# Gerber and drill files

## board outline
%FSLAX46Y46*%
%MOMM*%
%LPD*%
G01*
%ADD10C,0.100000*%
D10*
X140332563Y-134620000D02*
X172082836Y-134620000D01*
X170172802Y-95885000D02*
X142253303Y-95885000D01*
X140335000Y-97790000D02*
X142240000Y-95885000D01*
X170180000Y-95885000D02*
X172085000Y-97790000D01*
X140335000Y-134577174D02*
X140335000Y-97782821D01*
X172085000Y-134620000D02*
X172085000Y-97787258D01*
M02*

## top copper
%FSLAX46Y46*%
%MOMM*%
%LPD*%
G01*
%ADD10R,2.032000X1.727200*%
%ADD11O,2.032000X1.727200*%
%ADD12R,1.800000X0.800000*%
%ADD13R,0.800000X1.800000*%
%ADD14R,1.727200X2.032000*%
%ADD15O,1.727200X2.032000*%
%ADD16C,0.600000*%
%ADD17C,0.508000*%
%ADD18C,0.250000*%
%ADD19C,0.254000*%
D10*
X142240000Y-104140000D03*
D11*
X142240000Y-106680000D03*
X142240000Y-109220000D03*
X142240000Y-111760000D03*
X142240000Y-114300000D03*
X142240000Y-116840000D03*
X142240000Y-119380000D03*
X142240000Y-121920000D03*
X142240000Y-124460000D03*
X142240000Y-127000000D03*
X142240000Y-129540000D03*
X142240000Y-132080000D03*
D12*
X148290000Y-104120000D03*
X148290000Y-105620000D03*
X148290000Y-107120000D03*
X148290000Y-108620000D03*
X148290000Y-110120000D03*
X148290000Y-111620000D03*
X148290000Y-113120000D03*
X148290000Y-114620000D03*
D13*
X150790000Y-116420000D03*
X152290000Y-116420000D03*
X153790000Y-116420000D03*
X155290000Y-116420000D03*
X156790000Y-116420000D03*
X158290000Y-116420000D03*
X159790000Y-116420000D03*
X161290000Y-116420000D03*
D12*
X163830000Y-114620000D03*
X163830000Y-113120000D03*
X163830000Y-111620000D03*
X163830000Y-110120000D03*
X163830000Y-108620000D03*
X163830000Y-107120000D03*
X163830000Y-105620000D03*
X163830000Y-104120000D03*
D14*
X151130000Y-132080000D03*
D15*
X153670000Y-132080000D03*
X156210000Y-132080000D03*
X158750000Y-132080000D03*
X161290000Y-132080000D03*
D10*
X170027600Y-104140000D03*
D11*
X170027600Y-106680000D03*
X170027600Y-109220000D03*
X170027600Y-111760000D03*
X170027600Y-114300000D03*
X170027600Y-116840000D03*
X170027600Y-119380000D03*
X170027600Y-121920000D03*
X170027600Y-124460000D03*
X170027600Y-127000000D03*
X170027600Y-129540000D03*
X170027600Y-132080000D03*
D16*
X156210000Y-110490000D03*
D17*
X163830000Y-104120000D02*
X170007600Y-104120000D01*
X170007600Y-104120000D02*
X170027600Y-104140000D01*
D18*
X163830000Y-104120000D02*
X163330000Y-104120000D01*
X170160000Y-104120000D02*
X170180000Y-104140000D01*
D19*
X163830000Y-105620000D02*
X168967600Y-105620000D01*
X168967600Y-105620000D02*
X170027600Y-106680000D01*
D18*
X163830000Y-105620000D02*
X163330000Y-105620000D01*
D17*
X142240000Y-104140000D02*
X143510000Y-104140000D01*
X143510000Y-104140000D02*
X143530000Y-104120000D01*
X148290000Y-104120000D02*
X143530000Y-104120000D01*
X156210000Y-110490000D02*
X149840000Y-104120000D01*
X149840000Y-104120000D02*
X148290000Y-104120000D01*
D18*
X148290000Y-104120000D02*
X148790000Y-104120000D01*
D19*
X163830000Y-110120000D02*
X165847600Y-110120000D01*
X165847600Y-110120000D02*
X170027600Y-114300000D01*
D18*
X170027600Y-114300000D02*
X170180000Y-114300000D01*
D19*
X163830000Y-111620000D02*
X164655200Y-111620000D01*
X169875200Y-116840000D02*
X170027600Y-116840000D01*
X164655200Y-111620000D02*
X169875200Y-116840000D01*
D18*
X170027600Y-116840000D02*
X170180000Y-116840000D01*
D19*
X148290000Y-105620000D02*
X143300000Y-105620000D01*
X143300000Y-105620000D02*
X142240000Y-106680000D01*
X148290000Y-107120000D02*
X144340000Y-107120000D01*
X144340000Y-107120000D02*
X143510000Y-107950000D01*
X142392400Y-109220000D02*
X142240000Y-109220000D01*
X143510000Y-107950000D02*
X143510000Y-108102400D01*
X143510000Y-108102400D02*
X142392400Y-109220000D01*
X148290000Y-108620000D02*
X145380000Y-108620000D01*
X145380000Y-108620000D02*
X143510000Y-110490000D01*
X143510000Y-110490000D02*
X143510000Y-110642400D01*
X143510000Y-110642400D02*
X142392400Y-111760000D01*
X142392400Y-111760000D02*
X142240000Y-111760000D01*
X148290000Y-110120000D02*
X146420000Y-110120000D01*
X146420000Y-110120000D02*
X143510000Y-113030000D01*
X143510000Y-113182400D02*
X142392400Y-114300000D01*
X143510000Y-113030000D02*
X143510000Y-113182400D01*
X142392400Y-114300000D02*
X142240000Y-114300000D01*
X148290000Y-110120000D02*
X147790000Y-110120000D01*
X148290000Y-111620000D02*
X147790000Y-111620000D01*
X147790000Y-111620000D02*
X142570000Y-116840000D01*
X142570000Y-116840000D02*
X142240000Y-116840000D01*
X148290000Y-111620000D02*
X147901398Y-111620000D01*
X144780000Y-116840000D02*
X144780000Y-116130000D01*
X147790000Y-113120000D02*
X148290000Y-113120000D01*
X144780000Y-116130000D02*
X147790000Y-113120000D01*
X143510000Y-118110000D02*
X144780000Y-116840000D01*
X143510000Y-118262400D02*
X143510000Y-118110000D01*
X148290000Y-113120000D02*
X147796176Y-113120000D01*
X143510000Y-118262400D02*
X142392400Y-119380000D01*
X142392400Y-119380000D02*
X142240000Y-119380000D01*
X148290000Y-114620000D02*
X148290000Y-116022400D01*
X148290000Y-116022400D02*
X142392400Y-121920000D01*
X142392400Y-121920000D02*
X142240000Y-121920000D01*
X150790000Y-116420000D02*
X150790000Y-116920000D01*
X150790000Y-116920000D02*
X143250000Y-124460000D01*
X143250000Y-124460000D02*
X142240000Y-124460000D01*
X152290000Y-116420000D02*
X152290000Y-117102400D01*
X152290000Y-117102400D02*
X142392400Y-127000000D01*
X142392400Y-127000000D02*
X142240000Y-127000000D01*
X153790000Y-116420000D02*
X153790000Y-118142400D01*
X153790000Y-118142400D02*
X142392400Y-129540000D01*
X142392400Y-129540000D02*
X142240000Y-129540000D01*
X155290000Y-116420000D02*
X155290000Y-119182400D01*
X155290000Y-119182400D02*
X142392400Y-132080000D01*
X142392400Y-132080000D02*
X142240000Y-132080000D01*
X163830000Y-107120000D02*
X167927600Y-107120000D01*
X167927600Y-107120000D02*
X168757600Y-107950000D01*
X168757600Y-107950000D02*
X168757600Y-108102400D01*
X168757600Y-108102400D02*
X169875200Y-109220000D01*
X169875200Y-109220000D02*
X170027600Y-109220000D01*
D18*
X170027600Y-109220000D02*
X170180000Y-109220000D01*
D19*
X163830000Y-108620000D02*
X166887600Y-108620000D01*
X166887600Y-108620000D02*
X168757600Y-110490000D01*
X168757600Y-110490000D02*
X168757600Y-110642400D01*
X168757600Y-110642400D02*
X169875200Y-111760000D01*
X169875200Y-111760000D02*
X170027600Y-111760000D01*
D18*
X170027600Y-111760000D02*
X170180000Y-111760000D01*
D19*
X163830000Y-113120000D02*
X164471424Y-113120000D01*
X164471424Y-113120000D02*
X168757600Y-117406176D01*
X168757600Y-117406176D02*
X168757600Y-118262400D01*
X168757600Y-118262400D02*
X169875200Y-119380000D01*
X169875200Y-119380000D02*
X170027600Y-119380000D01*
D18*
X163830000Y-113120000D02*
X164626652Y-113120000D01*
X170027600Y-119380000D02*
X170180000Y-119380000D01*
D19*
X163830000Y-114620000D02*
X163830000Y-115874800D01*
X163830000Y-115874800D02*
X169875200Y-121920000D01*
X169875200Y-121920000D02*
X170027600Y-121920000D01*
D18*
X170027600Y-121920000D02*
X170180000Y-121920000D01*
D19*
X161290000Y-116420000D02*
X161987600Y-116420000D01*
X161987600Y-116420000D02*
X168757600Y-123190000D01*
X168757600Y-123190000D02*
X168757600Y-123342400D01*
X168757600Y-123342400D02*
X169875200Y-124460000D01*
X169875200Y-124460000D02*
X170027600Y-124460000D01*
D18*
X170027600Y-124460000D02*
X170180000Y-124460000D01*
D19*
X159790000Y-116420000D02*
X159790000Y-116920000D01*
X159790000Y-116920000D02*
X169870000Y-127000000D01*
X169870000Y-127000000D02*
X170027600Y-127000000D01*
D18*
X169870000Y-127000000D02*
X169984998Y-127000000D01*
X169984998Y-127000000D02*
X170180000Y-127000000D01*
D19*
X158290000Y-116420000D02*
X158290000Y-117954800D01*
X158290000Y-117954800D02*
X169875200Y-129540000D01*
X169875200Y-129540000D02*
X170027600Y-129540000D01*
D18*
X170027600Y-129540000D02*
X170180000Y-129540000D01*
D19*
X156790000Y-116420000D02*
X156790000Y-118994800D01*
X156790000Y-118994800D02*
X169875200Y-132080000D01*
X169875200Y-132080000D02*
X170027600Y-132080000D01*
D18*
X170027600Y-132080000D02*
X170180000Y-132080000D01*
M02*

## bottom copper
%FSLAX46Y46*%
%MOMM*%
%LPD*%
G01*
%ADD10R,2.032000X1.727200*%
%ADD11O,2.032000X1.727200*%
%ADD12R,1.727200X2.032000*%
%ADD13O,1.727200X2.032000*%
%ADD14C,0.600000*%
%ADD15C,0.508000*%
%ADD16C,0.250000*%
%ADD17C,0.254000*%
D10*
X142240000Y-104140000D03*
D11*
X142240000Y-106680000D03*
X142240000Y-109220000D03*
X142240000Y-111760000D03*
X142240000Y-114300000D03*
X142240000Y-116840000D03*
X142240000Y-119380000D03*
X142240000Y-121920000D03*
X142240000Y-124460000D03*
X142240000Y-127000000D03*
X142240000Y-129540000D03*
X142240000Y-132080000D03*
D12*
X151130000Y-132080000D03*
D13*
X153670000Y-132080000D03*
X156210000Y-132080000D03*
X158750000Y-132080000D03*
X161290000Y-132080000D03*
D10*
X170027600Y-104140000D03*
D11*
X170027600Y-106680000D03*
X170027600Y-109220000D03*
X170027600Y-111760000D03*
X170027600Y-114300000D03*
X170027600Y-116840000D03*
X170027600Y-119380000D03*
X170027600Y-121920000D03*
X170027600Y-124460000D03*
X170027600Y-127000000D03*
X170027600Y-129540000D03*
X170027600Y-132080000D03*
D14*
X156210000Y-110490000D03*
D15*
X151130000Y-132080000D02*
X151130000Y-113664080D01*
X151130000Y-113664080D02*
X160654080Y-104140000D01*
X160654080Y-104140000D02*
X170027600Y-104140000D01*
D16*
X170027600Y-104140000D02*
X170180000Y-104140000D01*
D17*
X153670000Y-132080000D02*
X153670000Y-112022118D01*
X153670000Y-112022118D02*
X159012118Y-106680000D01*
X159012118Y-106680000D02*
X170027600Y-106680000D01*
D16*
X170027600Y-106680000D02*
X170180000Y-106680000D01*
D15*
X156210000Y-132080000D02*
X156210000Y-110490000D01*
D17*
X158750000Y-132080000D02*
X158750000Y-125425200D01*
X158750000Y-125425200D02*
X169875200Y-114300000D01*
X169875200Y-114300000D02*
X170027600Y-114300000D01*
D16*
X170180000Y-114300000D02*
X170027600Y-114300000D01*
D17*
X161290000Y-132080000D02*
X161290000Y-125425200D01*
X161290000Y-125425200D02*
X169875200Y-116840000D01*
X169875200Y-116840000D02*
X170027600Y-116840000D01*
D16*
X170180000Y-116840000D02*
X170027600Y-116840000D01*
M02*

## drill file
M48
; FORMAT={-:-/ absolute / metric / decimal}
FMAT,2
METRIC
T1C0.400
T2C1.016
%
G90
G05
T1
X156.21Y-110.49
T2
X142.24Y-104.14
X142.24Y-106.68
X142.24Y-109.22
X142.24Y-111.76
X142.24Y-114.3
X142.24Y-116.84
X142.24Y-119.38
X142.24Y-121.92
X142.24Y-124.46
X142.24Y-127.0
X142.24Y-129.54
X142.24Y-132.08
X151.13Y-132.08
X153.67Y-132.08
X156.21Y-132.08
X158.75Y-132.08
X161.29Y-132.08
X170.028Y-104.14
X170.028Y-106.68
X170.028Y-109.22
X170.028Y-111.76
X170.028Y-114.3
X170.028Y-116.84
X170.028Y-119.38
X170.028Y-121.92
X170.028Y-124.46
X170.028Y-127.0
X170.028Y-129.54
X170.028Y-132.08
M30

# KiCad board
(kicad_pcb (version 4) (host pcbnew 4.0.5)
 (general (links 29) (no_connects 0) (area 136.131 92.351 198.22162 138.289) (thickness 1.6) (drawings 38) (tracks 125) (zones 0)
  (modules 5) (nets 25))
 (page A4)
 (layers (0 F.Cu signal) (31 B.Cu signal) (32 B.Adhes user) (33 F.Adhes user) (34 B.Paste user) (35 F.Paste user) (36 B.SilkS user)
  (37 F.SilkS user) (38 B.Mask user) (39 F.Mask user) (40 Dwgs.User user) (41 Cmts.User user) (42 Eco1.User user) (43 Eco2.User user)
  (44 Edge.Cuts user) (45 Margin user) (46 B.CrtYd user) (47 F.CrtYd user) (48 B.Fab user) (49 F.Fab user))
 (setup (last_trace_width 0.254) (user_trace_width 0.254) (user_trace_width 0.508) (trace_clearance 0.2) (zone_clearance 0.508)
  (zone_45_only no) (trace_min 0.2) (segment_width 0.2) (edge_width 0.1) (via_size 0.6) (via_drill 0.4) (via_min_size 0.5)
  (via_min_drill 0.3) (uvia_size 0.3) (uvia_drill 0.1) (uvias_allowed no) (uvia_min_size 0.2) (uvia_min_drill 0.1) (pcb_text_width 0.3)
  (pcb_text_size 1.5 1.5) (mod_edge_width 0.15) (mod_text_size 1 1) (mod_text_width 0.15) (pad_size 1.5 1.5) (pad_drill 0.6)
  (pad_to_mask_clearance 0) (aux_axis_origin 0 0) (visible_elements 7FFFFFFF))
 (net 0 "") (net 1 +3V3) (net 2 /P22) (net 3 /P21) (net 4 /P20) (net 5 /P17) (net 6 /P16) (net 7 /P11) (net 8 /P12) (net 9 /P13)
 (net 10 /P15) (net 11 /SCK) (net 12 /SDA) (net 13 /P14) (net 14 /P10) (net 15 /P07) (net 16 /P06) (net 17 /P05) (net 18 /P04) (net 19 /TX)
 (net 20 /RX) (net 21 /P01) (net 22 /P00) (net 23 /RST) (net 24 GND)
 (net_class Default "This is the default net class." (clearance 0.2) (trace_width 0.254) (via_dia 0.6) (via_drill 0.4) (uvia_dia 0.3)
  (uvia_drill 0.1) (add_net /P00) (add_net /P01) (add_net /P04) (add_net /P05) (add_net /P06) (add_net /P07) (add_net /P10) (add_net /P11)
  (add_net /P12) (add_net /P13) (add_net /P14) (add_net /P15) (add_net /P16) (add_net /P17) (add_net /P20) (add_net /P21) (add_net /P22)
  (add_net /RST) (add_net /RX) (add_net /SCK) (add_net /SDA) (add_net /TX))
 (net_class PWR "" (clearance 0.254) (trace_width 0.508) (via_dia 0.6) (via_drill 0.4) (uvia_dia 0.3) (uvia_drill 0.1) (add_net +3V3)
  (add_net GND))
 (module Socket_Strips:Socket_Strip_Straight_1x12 (layer F.Cu) (at 142.24 104.14 270)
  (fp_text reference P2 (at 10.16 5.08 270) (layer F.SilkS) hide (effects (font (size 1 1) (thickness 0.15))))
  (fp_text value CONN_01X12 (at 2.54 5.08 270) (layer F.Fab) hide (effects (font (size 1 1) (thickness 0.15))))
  (pad 1 thru_hole rect (at 0 0 270) (size 1.7272 2.032) (drill 1.016) (layers *.Cu *.Mask) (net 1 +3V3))
  (pad 2 thru_hole oval (at 2.54 0 270) (size 1.7272 2.032) (drill 1.016) (layers *.Cu *.Mask) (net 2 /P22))
  (pad 3 thru_hole oval (at 5.08 0 270) (size 1.7272 2.032) (drill 1.016) (layers *.Cu *.Mask) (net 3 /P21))
  (pad 4 thru_hole oval (at 7.62 0 270) (size 1.7272 2.032) (drill 1.016) (layers *.Cu *.Mask) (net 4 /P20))
  (pad 5 thru_hole oval (at 10.16 0 270) (size 1.7272 2.032) (drill 1.016) (layers *.Cu *.Mask) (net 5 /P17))
  (pad 6 thru_hole oval (at 12.7 0 270) (size 1.7272 2.032) (drill 1.016) (layers *.Cu *.Mask) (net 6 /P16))
  (pad 7 thru_hole oval (at 15.24 0 270) (size 1.7272 2.032) (drill 1.016) (layers *.Cu *.Mask) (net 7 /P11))
  (pad 8 thru_hole oval (at 17.78 0 270) (size 1.7272 2.032) (drill 1.016) (layers *.Cu *.Mask) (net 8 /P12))
  (pad 9 thru_hole oval (at 20.32 0 270) (size 1.7272 2.032) (drill 1.016) (layers *.Cu *.Mask) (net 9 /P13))
  (pad 10 thru_hole oval (at 22.86 0 270) (size 1.7272 2.032) (drill 1.016) (layers *.Cu *.Mask) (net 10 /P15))
  (pad 11 thru_hole oval (at 25.4 0 270) (size 1.7272 2.032) (drill 1.016) (layers *.Cu *.Mask) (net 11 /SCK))
  (pad 12 thru_hole oval (at 27.94 0 270) (size 1.7272 2.032) (drill 1.016) (layers *.Cu *.Mask) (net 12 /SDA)))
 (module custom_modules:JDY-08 (layer F.Cu) (at 148.59 96.52)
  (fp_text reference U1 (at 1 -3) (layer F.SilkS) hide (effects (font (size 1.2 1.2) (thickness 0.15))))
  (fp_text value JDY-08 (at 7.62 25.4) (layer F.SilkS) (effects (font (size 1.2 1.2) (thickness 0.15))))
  (pad 1 smd rect (at -0.3 7.6 90) (size 0.8 1.8) (layers F.Cu F.Paste F.Mask) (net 1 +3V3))
  (pad 2 smd rect (at -0.3 9.1 90) (size 0.8 1.8) (layers F.Cu F.Paste F.Mask) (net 2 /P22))
  (pad 3 smd rect (at -0.3 10.6 90) (size 0.8 1.8) (layers F.Cu F.Paste F.Mask) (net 3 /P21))
  (pad 4 smd rect (at -0.3 12.1 90) (size 0.8 1.8) (layers F.Cu F.Paste F.Mask) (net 4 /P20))
  (pad 5 smd rect (at -0.3 13.6 90) (size 0.8 1.8) (layers F.Cu F.Paste F.Mask) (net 5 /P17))
  (pad 6 smd rect (at -0.3 15.1 90) (size 0.8 1.8) (layers F.Cu F.Paste F.Mask) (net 6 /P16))
  (pad 7 smd rect (at -0.3 16.6 90) (size 0.8 1.8) (layers F.Cu F.Paste F.Mask) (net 7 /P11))
  (pad 8 smd rect (at -0.3 18.1 90) (size 0.8 1.8) (layers F.Cu F.Paste F.Mask) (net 8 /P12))
  (pad 9 smd rect (at 2.2 19.9) (size 0.8 1.8) (layers F.Cu F.Paste F.Mask) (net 9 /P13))
  (pad 10 smd rect (at 3.7 19.9) (size 0.8 1.8) (layers F.Cu F.Paste F.Mask) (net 10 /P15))
  (pad 11 smd rect (at 5.2 19.9) (size 0.8 1.8) (layers F.Cu F.Paste F.Mask) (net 11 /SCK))
  (pad 12 smd rect (at 6.7 19.9) (size 0.8 1.8) (layers F.Cu F.Paste F.Mask) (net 12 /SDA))
  (pad 13 smd rect (at 8.2 19.9) (size 0.8 1.8) (layers F.Cu F.Paste F.Mask) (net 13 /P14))
  (pad 14 smd rect (at 9.7 19.9) (size 0.8 1.8) (layers F.Cu F.Paste F.Mask) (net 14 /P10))
  (pad 15 smd rect (at 11.2 19.9) (size 0.8 1.8) (layers F.Cu F.Paste F.Mask) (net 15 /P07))
  (pad 16 smd rect (at 12.7 19.9) (size 0.8 1.8) (layers F.Cu F.Paste F.Mask) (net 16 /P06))
  (pad 17 smd rect (at 15.24 18.1 90) (size 0.8 1.8) (layers F.Cu F.Paste F.Mask) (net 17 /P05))
  (pad 18 smd rect (at 15.24 16.6 90) (size 0.8 1.8) (layers F.Cu F.Paste F.Mask) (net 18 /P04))
  (pad 19 smd rect (at 15.24 15.1 90) (size 0.8 1.8) (layers F.Cu F.Paste F.Mask) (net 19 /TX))
  (pad 20 smd rect (at 15.24 13.6 90) (size 0.8 1.8) (layers F.Cu F.Paste F.Mask) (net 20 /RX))
  (pad 21 smd rect (at 15.24 12.1 90) (size 0.8 1.8) (layers F.Cu F.Paste F.Mask) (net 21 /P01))
  (pad 22 smd rect (at 15.24 10.6 90) (size 0.8 1.8) (layers F.Cu F.Paste F.Mask) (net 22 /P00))
  (pad 23 smd rect (at 15.24 9.1 90) (size 0.8 1.8) (layers F.Cu F.Paste F.Mask) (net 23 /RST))
  (pad 24 smd rect (at 15.24 7.6 90) (size 0.8 1.8) (layers F.Cu F.Paste F.Mask) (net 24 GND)))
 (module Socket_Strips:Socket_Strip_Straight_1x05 (layer F.Cu) (at 151.13 132.08)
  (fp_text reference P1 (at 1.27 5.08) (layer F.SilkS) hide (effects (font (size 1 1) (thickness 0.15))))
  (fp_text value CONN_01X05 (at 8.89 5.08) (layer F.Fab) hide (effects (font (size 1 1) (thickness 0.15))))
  (pad 1 thru_hole rect (at 0 0) (size 1.7272 2.032) (drill 1.016) (layers *.Cu *.Mask) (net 24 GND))
  (pad 2 thru_hole oval (at 2.54 0) (size 1.7272 2.032) (drill 1.016) (layers *.Cu *.Mask) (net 23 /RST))
  (pad 3 thru_hole oval (at 5.08 0) (size 1.7272 2.032) (drill 1.016) (layers *.Cu *.Mask) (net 1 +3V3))
  (pad 4 thru_hole oval (at 7.62 0) (size 1.7272 2.032) (drill 1.016) (layers *.Cu *.Mask) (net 20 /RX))
  (pad 5 thru_hole oval (at 10.16 0) (size 1.7272 2.032) (drill 1.016) (layers *.Cu *.Mask) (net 19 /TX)))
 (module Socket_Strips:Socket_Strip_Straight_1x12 (layer F.Cu) (at 170.0276 104.14 270)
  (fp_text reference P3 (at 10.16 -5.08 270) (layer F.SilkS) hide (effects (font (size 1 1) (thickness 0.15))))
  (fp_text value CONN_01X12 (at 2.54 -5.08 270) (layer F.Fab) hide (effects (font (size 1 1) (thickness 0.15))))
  (pad 1 thru_hole rect (at 0 0 270) (size 1.7272 2.032) (drill 1.016) (layers *.Cu *.Mask) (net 24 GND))
  (pad 2 thru_hole oval (at 2.54 0 270) (size 1.7272 2.032) (drill 1.016) (layers *.Cu *.Mask) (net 23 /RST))
  (pad 3 thru_hole oval (at 5.08 0 270) (size 1.7272 2.032) (drill 1.016) (layers *.Cu *.Mask) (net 22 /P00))
  (pad 4 thru_hole oval (at 7.62 0 270) (size 1.7272 2.032) (drill 1.016) (layers *.Cu *.Mask) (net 21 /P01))
  (pad 5 thru_hole oval (at 10.16 0 270) (size 1.7272 2.032) (drill 1.016) (layers *.Cu *.Mask) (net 20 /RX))
  (pad 6 thru_hole oval (at 12.7 0 270) (size 1.7272 2.032) (drill 1.016) (layers *.Cu *.Mask) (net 19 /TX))
  (pad 7 thru_hole oval (at 15.24 0 270) (size 1.7272 2.032) (drill 1.016) (layers *.Cu *.Mask) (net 18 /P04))
  (pad 8 thru_hole oval (at 17.78 0 270) (size 1.7272 2.032) (drill 1.016) (layers *.Cu *.Mask) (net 17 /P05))
  (pad 9 thru_hole oval (at 20.32 0 270) (size 1.7272 2.032) (drill 1.016) (layers *.Cu *.Mask) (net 16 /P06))
  (pad 10 thru_hole oval (at 22.86 0 270) (size 1.7272 2.032) (drill 1.016) (layers *.Cu *.Mask) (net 15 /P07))
  (pad 11 thru_hole oval (at 25.4 0 270) (size 1.7272 2.032) (drill 1.016) (layers *.Cu *.Mask) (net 14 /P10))
  (pad 12 thru_hole oval (at 27.94 0 270) (size 1.7272 2.032) (drill 1.016) (layers *.Cu *.Mask) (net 13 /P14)))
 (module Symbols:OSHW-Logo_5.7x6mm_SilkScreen (layer F.Cu) (at 149.86 124.46)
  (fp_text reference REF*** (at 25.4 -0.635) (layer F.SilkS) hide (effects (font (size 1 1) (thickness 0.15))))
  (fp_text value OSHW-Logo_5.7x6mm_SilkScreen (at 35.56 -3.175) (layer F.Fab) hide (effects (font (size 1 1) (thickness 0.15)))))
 (gr_line (start 140.332563 134.62) (end 172.082836 134.62) (layer Edge.Cuts) (width 0.1))
 (gr_line (start 170.172802 95.885) (end 142.253303 95.885) (layer Edge.Cuts) (width 0.1))
 (gr_line (start 140.335 97.79) (end 142.24 95.885) (layer Edge.Cuts) (width 0.1))
 (gr_line (start 170.18 95.885) (end 172.085 97.79) (layer Edge.Cuts) (width 0.1))
 (gr_line (start 140.335 134.577174) (end 140.335 97.782821) (layer Edge.Cuts) (width 0.1))
 (gr_line (start 172.085 134.62) (end 172.085 97.787258) (layer Edge.Cuts) (width 0.1))
 (segment (start 151.13 132.08) (end 151.13 113.66408) (width 0.508) (layer B.Cu) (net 24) (status 10))
 (segment (start 151.13 113.66408) (end 160.65408 104.14) (width 0.508) (layer B.Cu) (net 24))
 (segment (start 160.65408 104.14) (end 170.0276 104.14) (width 0.508) (layer B.Cu) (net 24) (status 20))
 (segment (start 163.83 104.12) (end 170.0076 104.12) (width 0.508) (layer F.Cu) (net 24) (status 30))
 (segment (start 170.0076 104.12) (end 170.0276 104.14) (width 0.508) (layer F.Cu) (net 24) (status 30))
 (segment (start 170.0276 104.14) (end 170.18 104.14) (width 0.25) (layer B.Cu) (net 24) (status 30))
 (segment (start 163.83 104.12) (end 163.33 104.12) (width 0.25) (layer F.Cu) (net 24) (status 30))
 (segment (start 170.16 104.12) (end 170.18 104.14) (width 0.25) (layer F.Cu) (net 24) (status 30))
 (segment (start 153.67 132.08) (end 153.67 112.022118) (width 0.254) (layer B.Cu) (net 23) (status 10))
 (segment (start 153.67 112.022118) (end 159.012118 106.68) (width 0.254) (layer B.Cu) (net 23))
 (segment (start 159.012118 106.68) (end 170.0276 106.68) (width 0.254) (layer B.Cu) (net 23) (status 20))
 (segment (start 163.83 105.62) (end 168.9676 105.62) (width 0.254) (layer F.Cu) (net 23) (status 10))
 (segment (start 168.9676 105.62) (end 170.0276 106.68) (width 0.254) (layer F.Cu) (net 23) (status 20))
 (segment (start 170.0276 106.68) (end 170.18 106.68) (width 0.25) (layer B.Cu) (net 23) (status 30))
 (segment (start 163.83 105.62) (end 163.33 105.62) (width 0.25) (layer F.Cu) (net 23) (status 30))
 (segment (start 142.24 104.14) (end 143.51 104.14) (width 0.508) (layer F.Cu) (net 1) (status 10))
 (segment (start 143.51 104.14) (end 143.53 104.12) (width 0.508) (layer F.Cu) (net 1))
 (segment (start 148.29 104.12) (end 143.53 104.12) (width 0.508) (layer F.Cu) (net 1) (status 10))
 (segment (start 156.21 110.49) (end 149.84 104.12) (width 0.508) (layer F.Cu) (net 1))
 (segment (start 149.84 104.12) (end 148.29 104.12) (width 0.508) (layer F.Cu) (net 1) (status 20))
 (segment (start 156.21 132.08) (end 156.21 110.49) (width 0.508) (layer B.Cu) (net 1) (status 10))
 (via (at 156.21 110.49) (size 0.6) (drill 0.4) (layers F.Cu B.Cu) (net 1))
 (segment (start 148.29 104.12) (end 148.79 104.12) (width 0.25) (layer F.Cu) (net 1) (status 30))
 (segment (start 158.75 132.08) (end 158.75 125.4252) (width 0.254) (layer B.Cu) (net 20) (status 10))
 (segment (start 158.75 125.4252) (end 169.8752 114.3) (width 0.254) (layer B.Cu) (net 20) (status 20))
 (segment (start 169.8752 114.3) (end 170.0276 114.3) (width 0.254) (layer B.Cu) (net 20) (status 30))
 (segment (start 163.83 110.12) (end 165.8476 110.12) (width 0.254) (layer F.Cu) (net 20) (status 10))
 (segment (start 165.8476 110.12) (end 170.0276 114.3) (width 0.254) (layer F.Cu) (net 20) (status 20))
 (segment (start 170.18 114.3) (end 170.0276 114.3) (width 0.25) (layer B.Cu) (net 20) (status 30))
 (segment (start 170.0276 114.3) (end 170.18 114.3) (width 0.25) (layer F.Cu) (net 20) (status 30))
 (segment (start 161.29 132.08) (end 161.29 125.4252) (width 0.254) (layer B.Cu) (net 19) (status 10))
 (segment (start 161.29 125.4252) (end 169.8752 116.84) (width 0.254) (layer B.Cu) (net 19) (status 20))
 (segment (start 169.8752 116.84) (end 170.0276 116.84) (width 0.254) (layer B.Cu) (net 19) (status 30))
 (segment (start 163.83 111.62) (end 164.6552 111.62) (width 0.254) (layer F.Cu) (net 19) (status 30))
 (segment (start 169.8752 116.84) (end 170.0276 116.84) (width 0.254) (layer F.Cu) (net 19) (status 30))
 (segment (start 164.6552 111.62) (end 169.8752 116.84) (width 0.254) (layer F.Cu) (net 19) (status 30))
 (segment (start 170.18 116.84) (end 170.0276 116.84) (width 0.25) (layer B.Cu) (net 19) (status 30))
 (segment (start 170.0276 116.84) (end 170.18 116.84) (width 0.25) (layer F.Cu) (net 19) (status 30))
 (segment (start 148.29 105.62) (end 143.3 105.62) (width 0.254) (layer F.Cu) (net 2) (status 10))
 (segment (start 143.3 105.62) (end 142.24 106.68) (width 0.254) (layer F.Cu) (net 2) (status 20))
 (segment (start 148.29 107.12) (end 144.34 107.12) (width 0.254) (layer F.Cu) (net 3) (status 10))
 (segment (start 144.34 107.12) (end 143.51 107.95) (width 0.254) (layer F.Cu) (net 3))
 (segment (start 142.3924 109.22) (end 142.24 109.22) (width 0.254) (layer F.Cu) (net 3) (status 30))
 (segment (start 143.51 107.95) (end 143.51 108.1024) (width 0.254) (layer F.Cu) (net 3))
 (segment (start 143.51 108.1024) (end 142.3924 109.22) (width 0.254) (layer F.Cu) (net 3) (status 20))
 (segment (start 148.29 108.62) (end 145.38 108.62) (width 0.254) (layer F.Cu) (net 4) (status 10))
 (segment (start 145.38 108.62) (end 143.51 110.49) (width 0.254) (layer F.Cu) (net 4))
 (segment (start 143.51 110.49) (end 143.51 110.6424) (width 0.254) (layer F.Cu) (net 4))
 (segment (start 143.51 110.6424) (end 142.3924 111.76) (width 0.254) (layer F.Cu) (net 4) (status 20))
 (segment (start 142.3924 111.76) (end 142.24 111.76) (width 0.254) (layer F.Cu) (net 4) (status 30))
 (segment (start 148.29 110.12) (end 146.42 110.12) (width 0.254) (layer F.Cu) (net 5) (status 10))
 (segment (start 146.42 110.12) (end 143.51 113.03) (width 0.254) (layer F.Cu) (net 5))
 (segment (start 143.51 113.1824) (end 142.3924 114.3) (width 0.254) (layer F.Cu) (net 5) (status 20))
 (segment (start 143.51 113.03) (end 143.51 113.1824) (width 0.254) (layer F.Cu) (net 5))
 (segment (start 142.3924 114.3) (end 142.24 114.3) (width 0.254) (layer F.Cu) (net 5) (status 30))
 (segment (start 148.29 110.12) (end 147.79 110.12) (width 0.254) (layer F.Cu) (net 5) (status 30))
 (segment (start 148.29 111.62) (end 147.79 111.62) (width 0.254) (layer F.Cu) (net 6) (status 30))
 (segment (start 147.79 111.62) (end 142.57 116.84) (width 0.254) (layer F.Cu) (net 6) (status 30))
 (segment (start 142.57 116.84) (end 142.24 116.84) (width 0.254) (layer F.Cu) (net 6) (status 30))
 (segment (start 148.29 111.62) (end 147.901398 111.62) (width 0.254) (layer F.Cu) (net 6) (status 30))
 (segment (start 144.78 116.84) (end 144.78 116.13) (width 0.254) (layer F.Cu) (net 7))
 (segment (start 147.79 113.12) (end 148.29 113.12) (width 0.254) (layer F.Cu) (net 7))
 (segment (start 144.78 116.13) (end 147.79 113.12) (width 0.254) (layer F.Cu) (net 7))
 (segment (start 143.51 118.11) (end 144.78 116.84) (width 0.254) (layer F.Cu) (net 7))
 (segment (start 143.51 118.2624) (end 143.51 118.11) (width 0.254) (layer F.Cu) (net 7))
 (segment (start 148.29 113.12) (end 147.796176 113.12) (width 0.254) (layer F.Cu) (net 7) (status 30))
 (segment (start 143.51 118.2624) (end 142.3924 119.38) (width 0.254) (layer F.Cu) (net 7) (status 20))
 (segment (start 142.3924 119.38) (end 142.24 119.38) (width 0.254) (layer F.Cu) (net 7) (status 30))
 (segment (start 148.29 114.62) (end 148.29 116.0224) (width 0.254) (layer F.Cu) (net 8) (status 10))
 (segment (start 148.29 116.0224) (end 142.3924 121.92) (width 0.254) (layer F.Cu) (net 8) (status 20))
 (segment (start 142.3924 121.92) (end 142.24 121.92) (width 0.254) (layer F.Cu) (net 8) (status 30))
 (segment (start 150.79 116.42) (end 150.79 116.92) (width 0.254) (layer F.Cu) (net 9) (status 30))
 (segment (start 150.79 116.92) (end 143.25 124.46) (width 0.254) (layer F.Cu) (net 9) (status 30))
 (segment (start 143.25 124.46) (end 142.24 124.46) (width 0.254) (layer F.Cu) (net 9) (status 30))
 (segment (start 152.29 116.42) (end 152.29 117.1024) (width 0.254) (layer F.Cu) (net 10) (status 30))
 (segment (start 152.29 117.1024) (end 142.3924 127) (width 0.254) (layer F.Cu) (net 10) (status 30))
 (segment (start 142.3924 127) (end 142.24 127) (width 0.254) (layer F.Cu) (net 10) (status 30))
 (segment (start 153.79 116.42) (end 153.79 118.1424) (width 0.254) (layer F.Cu) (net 11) (status 10))
 (segment (start 153.79 118.1424) (end 142.3924 129.54) (width 0.254) (layer F.Cu) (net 11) (status 20))
 (segment (start 142.3924 129.54) (end 142.24 129.54) (width 0.254) (layer F.Cu) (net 11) (status 30))
 (segment (start 155.29 116.42) (end 155.29 119.1824) (width 0.254) (layer F.Cu) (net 12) (status 10))
 (segment (start 155.29 119.1824) (end 142.3924 132.08) (width 0.254) (layer F.Cu) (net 12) (status 20))
 (segment (start 142.3924 132.08) (end 142.24 132.08) (width 0.254) (layer F.Cu) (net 12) (status 30))
 (segment (start 163.83 107.12) (end 167.9276 107.12) (width 0.254) (layer F.Cu) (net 22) (status 10))
 (segment (start 167.9276 107.12) (end 168.7576 107.95) (width 0.254) (layer F.Cu) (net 22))
 (segment (start 168.7576 107.95) (end 168.7576 108.1024) (width 0.254) (layer F.Cu) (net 22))
 (segment (start 168.7576 108.1024) (end 169.8752 109.22) (width 0.254) (layer F.Cu) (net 22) (status 20))
 (segment (start 169.8752 109.22) (end 170.0276 109.22) (width 0.254) (layer F.Cu) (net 22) (status 30))
 (segment (start 170.0276 109.22) (end 170.18 109.22) (width 0.25) (layer F.Cu) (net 22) (status 30))
 (segment (start 163.83 108.62) (end 166.8876 108.62) (width 0.254) (layer F.Cu) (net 21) (status 10))
 (segment (start 166.8876 108.62) (end 168.7576 110.49) (width 0.254) (layer F.Cu) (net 21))
 (segment (start 168.7576 110.49) (end 168.7576 110.6424) (width 0.254) (layer F.Cu) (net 21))
 (segment (start 168.7576 110.6424) (end 169.8752 111.76) (width 0.254) (layer F.Cu) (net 21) (status 20))
 (segment (start 169.8752 111.76) (end 170.0276 111.76) (width 0.254) (layer F.Cu) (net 21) (status 30))
 (segment (start 170.0276 111.76) (end 170.18 111.76) (width 0.25) (layer F.Cu) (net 21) (status 30))
 (segment (start 163.83 113.12) (end 164.471424 113.12) (width 0.254) (layer F.Cu) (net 18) (status 30))
 (segment (start 164.471424 113.12) (end 168.7576 117.406176) (width 0.254) (layer F.Cu) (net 18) (status 10))
 (segment (start 168.7576 117.406176) (end 168.7576 118.2624) (width 0.254) (layer F.Cu) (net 18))
 (segment (start 168.7576 118.2624) (end 169.8752 119.38) (width 0.254) (layer F.Cu) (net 18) (status 20))
 (segment (start 169.8752 119.38) (end 170.0276 119.38) (width 0.254) (layer F.Cu) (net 18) (status 30))
 (segment (start 163.83 113.12) (end 164.626652 113.12) (width 0.25) (layer F.Cu) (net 18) (status 30))
 (segment (start 170.0276 119.38) (end 170.18 119.38) (width 0.25) (layer F.Cu) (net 18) (status 30))
 (segment (start 163.83 114.62) (end 163.83 115.8748) (width 0.254) (layer F.Cu) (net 17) (status 10))
 (segment (start 163.83 115.8748) (end 169.8752 121.92) (width 0.254) (layer F.Cu) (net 17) (status 20))
 (segment (start 169.8752 121.92) (end 170.0276 121.92) (width 0.254) (layer F.Cu) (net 17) (status 30))
 (segment (start 170.0276 121.92) (end 170.18 121.92) (width 0.25) (layer F.Cu) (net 17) (status 30))
 (segment (start 161.29 116.42) (end 161.9876 116.42) (width 0.254) (layer F.Cu) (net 16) (status 10))
 (segment (start 161.9876 116.42) (end 168.7576 123.19) (width 0.254) (layer F.Cu) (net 16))
 (segment (start 168.7576 123.19) (end 168.7576 123.3424) (width 0.254) (layer F.Cu) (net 16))
 (segment (start 168.7576 123.3424) (end 169.8752 124.46) (width 0.254) (layer F.Cu) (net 16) (status 20))
 (segment (start 169.8752 124.46) (end 170.0276 124.46) (width 0.254) (layer F.Cu) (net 16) (status 30))
 (segment (start 170.0276 124.46) (end 170.18 124.46) (width 0.25) (layer F.Cu) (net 16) (status 30))
 (segment (start 159.79 116.42) (end 159.79 116.92) (width 0.254) (layer F.Cu) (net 15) (status 30))
 (segment (start 159.79 116.92) (end 169.87 127) (width 0.254) (layer F.Cu) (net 15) (status 30))
 (segment (start 169.87 127) (end 170.0276 127) (width 0.254) (layer F.Cu) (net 15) (status 30))
 (segment (start 169.87 127) (end 169.984998 127) (width 0.25) (layer F.Cu) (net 15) (status 30))
 (segment (start 169.984998 127) (end 170.18 127) (width 0.25) (layer F.Cu) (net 15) (status 30))
 (segment (start 158.29 116.42) (end 158.29 117.9548) (width 0.254) (layer F.Cu) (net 14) (status 10))
 (segment (start 158.29 117.9548) (end 169.8752 129.54) (width 0.254) (layer F.Cu) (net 14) (status 20))
 (segment (start 169.8752 129.54) (end 170.0276 129.54) (width 0.254) (layer F.Cu) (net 14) (status 30))
 (segment (start 170.0276 129.54) (end 170.18 129.54) (width 0.25) (layer F.Cu) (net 14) (status 30))
 (segment (start 156.79 116.42) (end 156.79 118.9948) (width 0.254) (layer F.Cu) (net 13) (status 10))
 (segment (start 156.79 118.9948) (end 169.8752 132.08) (width 0.254) (layer F.Cu) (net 13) (status 20))
 (segment (start 169.8752 132.08) (end 170.0276 132.08) (width 0.254) (layer F.Cu) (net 13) (status 30))
 (segment (start 170.0276 132.08) (end 170.18 132.08) (width 0.25) (layer F.Cu) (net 13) (status 30)))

